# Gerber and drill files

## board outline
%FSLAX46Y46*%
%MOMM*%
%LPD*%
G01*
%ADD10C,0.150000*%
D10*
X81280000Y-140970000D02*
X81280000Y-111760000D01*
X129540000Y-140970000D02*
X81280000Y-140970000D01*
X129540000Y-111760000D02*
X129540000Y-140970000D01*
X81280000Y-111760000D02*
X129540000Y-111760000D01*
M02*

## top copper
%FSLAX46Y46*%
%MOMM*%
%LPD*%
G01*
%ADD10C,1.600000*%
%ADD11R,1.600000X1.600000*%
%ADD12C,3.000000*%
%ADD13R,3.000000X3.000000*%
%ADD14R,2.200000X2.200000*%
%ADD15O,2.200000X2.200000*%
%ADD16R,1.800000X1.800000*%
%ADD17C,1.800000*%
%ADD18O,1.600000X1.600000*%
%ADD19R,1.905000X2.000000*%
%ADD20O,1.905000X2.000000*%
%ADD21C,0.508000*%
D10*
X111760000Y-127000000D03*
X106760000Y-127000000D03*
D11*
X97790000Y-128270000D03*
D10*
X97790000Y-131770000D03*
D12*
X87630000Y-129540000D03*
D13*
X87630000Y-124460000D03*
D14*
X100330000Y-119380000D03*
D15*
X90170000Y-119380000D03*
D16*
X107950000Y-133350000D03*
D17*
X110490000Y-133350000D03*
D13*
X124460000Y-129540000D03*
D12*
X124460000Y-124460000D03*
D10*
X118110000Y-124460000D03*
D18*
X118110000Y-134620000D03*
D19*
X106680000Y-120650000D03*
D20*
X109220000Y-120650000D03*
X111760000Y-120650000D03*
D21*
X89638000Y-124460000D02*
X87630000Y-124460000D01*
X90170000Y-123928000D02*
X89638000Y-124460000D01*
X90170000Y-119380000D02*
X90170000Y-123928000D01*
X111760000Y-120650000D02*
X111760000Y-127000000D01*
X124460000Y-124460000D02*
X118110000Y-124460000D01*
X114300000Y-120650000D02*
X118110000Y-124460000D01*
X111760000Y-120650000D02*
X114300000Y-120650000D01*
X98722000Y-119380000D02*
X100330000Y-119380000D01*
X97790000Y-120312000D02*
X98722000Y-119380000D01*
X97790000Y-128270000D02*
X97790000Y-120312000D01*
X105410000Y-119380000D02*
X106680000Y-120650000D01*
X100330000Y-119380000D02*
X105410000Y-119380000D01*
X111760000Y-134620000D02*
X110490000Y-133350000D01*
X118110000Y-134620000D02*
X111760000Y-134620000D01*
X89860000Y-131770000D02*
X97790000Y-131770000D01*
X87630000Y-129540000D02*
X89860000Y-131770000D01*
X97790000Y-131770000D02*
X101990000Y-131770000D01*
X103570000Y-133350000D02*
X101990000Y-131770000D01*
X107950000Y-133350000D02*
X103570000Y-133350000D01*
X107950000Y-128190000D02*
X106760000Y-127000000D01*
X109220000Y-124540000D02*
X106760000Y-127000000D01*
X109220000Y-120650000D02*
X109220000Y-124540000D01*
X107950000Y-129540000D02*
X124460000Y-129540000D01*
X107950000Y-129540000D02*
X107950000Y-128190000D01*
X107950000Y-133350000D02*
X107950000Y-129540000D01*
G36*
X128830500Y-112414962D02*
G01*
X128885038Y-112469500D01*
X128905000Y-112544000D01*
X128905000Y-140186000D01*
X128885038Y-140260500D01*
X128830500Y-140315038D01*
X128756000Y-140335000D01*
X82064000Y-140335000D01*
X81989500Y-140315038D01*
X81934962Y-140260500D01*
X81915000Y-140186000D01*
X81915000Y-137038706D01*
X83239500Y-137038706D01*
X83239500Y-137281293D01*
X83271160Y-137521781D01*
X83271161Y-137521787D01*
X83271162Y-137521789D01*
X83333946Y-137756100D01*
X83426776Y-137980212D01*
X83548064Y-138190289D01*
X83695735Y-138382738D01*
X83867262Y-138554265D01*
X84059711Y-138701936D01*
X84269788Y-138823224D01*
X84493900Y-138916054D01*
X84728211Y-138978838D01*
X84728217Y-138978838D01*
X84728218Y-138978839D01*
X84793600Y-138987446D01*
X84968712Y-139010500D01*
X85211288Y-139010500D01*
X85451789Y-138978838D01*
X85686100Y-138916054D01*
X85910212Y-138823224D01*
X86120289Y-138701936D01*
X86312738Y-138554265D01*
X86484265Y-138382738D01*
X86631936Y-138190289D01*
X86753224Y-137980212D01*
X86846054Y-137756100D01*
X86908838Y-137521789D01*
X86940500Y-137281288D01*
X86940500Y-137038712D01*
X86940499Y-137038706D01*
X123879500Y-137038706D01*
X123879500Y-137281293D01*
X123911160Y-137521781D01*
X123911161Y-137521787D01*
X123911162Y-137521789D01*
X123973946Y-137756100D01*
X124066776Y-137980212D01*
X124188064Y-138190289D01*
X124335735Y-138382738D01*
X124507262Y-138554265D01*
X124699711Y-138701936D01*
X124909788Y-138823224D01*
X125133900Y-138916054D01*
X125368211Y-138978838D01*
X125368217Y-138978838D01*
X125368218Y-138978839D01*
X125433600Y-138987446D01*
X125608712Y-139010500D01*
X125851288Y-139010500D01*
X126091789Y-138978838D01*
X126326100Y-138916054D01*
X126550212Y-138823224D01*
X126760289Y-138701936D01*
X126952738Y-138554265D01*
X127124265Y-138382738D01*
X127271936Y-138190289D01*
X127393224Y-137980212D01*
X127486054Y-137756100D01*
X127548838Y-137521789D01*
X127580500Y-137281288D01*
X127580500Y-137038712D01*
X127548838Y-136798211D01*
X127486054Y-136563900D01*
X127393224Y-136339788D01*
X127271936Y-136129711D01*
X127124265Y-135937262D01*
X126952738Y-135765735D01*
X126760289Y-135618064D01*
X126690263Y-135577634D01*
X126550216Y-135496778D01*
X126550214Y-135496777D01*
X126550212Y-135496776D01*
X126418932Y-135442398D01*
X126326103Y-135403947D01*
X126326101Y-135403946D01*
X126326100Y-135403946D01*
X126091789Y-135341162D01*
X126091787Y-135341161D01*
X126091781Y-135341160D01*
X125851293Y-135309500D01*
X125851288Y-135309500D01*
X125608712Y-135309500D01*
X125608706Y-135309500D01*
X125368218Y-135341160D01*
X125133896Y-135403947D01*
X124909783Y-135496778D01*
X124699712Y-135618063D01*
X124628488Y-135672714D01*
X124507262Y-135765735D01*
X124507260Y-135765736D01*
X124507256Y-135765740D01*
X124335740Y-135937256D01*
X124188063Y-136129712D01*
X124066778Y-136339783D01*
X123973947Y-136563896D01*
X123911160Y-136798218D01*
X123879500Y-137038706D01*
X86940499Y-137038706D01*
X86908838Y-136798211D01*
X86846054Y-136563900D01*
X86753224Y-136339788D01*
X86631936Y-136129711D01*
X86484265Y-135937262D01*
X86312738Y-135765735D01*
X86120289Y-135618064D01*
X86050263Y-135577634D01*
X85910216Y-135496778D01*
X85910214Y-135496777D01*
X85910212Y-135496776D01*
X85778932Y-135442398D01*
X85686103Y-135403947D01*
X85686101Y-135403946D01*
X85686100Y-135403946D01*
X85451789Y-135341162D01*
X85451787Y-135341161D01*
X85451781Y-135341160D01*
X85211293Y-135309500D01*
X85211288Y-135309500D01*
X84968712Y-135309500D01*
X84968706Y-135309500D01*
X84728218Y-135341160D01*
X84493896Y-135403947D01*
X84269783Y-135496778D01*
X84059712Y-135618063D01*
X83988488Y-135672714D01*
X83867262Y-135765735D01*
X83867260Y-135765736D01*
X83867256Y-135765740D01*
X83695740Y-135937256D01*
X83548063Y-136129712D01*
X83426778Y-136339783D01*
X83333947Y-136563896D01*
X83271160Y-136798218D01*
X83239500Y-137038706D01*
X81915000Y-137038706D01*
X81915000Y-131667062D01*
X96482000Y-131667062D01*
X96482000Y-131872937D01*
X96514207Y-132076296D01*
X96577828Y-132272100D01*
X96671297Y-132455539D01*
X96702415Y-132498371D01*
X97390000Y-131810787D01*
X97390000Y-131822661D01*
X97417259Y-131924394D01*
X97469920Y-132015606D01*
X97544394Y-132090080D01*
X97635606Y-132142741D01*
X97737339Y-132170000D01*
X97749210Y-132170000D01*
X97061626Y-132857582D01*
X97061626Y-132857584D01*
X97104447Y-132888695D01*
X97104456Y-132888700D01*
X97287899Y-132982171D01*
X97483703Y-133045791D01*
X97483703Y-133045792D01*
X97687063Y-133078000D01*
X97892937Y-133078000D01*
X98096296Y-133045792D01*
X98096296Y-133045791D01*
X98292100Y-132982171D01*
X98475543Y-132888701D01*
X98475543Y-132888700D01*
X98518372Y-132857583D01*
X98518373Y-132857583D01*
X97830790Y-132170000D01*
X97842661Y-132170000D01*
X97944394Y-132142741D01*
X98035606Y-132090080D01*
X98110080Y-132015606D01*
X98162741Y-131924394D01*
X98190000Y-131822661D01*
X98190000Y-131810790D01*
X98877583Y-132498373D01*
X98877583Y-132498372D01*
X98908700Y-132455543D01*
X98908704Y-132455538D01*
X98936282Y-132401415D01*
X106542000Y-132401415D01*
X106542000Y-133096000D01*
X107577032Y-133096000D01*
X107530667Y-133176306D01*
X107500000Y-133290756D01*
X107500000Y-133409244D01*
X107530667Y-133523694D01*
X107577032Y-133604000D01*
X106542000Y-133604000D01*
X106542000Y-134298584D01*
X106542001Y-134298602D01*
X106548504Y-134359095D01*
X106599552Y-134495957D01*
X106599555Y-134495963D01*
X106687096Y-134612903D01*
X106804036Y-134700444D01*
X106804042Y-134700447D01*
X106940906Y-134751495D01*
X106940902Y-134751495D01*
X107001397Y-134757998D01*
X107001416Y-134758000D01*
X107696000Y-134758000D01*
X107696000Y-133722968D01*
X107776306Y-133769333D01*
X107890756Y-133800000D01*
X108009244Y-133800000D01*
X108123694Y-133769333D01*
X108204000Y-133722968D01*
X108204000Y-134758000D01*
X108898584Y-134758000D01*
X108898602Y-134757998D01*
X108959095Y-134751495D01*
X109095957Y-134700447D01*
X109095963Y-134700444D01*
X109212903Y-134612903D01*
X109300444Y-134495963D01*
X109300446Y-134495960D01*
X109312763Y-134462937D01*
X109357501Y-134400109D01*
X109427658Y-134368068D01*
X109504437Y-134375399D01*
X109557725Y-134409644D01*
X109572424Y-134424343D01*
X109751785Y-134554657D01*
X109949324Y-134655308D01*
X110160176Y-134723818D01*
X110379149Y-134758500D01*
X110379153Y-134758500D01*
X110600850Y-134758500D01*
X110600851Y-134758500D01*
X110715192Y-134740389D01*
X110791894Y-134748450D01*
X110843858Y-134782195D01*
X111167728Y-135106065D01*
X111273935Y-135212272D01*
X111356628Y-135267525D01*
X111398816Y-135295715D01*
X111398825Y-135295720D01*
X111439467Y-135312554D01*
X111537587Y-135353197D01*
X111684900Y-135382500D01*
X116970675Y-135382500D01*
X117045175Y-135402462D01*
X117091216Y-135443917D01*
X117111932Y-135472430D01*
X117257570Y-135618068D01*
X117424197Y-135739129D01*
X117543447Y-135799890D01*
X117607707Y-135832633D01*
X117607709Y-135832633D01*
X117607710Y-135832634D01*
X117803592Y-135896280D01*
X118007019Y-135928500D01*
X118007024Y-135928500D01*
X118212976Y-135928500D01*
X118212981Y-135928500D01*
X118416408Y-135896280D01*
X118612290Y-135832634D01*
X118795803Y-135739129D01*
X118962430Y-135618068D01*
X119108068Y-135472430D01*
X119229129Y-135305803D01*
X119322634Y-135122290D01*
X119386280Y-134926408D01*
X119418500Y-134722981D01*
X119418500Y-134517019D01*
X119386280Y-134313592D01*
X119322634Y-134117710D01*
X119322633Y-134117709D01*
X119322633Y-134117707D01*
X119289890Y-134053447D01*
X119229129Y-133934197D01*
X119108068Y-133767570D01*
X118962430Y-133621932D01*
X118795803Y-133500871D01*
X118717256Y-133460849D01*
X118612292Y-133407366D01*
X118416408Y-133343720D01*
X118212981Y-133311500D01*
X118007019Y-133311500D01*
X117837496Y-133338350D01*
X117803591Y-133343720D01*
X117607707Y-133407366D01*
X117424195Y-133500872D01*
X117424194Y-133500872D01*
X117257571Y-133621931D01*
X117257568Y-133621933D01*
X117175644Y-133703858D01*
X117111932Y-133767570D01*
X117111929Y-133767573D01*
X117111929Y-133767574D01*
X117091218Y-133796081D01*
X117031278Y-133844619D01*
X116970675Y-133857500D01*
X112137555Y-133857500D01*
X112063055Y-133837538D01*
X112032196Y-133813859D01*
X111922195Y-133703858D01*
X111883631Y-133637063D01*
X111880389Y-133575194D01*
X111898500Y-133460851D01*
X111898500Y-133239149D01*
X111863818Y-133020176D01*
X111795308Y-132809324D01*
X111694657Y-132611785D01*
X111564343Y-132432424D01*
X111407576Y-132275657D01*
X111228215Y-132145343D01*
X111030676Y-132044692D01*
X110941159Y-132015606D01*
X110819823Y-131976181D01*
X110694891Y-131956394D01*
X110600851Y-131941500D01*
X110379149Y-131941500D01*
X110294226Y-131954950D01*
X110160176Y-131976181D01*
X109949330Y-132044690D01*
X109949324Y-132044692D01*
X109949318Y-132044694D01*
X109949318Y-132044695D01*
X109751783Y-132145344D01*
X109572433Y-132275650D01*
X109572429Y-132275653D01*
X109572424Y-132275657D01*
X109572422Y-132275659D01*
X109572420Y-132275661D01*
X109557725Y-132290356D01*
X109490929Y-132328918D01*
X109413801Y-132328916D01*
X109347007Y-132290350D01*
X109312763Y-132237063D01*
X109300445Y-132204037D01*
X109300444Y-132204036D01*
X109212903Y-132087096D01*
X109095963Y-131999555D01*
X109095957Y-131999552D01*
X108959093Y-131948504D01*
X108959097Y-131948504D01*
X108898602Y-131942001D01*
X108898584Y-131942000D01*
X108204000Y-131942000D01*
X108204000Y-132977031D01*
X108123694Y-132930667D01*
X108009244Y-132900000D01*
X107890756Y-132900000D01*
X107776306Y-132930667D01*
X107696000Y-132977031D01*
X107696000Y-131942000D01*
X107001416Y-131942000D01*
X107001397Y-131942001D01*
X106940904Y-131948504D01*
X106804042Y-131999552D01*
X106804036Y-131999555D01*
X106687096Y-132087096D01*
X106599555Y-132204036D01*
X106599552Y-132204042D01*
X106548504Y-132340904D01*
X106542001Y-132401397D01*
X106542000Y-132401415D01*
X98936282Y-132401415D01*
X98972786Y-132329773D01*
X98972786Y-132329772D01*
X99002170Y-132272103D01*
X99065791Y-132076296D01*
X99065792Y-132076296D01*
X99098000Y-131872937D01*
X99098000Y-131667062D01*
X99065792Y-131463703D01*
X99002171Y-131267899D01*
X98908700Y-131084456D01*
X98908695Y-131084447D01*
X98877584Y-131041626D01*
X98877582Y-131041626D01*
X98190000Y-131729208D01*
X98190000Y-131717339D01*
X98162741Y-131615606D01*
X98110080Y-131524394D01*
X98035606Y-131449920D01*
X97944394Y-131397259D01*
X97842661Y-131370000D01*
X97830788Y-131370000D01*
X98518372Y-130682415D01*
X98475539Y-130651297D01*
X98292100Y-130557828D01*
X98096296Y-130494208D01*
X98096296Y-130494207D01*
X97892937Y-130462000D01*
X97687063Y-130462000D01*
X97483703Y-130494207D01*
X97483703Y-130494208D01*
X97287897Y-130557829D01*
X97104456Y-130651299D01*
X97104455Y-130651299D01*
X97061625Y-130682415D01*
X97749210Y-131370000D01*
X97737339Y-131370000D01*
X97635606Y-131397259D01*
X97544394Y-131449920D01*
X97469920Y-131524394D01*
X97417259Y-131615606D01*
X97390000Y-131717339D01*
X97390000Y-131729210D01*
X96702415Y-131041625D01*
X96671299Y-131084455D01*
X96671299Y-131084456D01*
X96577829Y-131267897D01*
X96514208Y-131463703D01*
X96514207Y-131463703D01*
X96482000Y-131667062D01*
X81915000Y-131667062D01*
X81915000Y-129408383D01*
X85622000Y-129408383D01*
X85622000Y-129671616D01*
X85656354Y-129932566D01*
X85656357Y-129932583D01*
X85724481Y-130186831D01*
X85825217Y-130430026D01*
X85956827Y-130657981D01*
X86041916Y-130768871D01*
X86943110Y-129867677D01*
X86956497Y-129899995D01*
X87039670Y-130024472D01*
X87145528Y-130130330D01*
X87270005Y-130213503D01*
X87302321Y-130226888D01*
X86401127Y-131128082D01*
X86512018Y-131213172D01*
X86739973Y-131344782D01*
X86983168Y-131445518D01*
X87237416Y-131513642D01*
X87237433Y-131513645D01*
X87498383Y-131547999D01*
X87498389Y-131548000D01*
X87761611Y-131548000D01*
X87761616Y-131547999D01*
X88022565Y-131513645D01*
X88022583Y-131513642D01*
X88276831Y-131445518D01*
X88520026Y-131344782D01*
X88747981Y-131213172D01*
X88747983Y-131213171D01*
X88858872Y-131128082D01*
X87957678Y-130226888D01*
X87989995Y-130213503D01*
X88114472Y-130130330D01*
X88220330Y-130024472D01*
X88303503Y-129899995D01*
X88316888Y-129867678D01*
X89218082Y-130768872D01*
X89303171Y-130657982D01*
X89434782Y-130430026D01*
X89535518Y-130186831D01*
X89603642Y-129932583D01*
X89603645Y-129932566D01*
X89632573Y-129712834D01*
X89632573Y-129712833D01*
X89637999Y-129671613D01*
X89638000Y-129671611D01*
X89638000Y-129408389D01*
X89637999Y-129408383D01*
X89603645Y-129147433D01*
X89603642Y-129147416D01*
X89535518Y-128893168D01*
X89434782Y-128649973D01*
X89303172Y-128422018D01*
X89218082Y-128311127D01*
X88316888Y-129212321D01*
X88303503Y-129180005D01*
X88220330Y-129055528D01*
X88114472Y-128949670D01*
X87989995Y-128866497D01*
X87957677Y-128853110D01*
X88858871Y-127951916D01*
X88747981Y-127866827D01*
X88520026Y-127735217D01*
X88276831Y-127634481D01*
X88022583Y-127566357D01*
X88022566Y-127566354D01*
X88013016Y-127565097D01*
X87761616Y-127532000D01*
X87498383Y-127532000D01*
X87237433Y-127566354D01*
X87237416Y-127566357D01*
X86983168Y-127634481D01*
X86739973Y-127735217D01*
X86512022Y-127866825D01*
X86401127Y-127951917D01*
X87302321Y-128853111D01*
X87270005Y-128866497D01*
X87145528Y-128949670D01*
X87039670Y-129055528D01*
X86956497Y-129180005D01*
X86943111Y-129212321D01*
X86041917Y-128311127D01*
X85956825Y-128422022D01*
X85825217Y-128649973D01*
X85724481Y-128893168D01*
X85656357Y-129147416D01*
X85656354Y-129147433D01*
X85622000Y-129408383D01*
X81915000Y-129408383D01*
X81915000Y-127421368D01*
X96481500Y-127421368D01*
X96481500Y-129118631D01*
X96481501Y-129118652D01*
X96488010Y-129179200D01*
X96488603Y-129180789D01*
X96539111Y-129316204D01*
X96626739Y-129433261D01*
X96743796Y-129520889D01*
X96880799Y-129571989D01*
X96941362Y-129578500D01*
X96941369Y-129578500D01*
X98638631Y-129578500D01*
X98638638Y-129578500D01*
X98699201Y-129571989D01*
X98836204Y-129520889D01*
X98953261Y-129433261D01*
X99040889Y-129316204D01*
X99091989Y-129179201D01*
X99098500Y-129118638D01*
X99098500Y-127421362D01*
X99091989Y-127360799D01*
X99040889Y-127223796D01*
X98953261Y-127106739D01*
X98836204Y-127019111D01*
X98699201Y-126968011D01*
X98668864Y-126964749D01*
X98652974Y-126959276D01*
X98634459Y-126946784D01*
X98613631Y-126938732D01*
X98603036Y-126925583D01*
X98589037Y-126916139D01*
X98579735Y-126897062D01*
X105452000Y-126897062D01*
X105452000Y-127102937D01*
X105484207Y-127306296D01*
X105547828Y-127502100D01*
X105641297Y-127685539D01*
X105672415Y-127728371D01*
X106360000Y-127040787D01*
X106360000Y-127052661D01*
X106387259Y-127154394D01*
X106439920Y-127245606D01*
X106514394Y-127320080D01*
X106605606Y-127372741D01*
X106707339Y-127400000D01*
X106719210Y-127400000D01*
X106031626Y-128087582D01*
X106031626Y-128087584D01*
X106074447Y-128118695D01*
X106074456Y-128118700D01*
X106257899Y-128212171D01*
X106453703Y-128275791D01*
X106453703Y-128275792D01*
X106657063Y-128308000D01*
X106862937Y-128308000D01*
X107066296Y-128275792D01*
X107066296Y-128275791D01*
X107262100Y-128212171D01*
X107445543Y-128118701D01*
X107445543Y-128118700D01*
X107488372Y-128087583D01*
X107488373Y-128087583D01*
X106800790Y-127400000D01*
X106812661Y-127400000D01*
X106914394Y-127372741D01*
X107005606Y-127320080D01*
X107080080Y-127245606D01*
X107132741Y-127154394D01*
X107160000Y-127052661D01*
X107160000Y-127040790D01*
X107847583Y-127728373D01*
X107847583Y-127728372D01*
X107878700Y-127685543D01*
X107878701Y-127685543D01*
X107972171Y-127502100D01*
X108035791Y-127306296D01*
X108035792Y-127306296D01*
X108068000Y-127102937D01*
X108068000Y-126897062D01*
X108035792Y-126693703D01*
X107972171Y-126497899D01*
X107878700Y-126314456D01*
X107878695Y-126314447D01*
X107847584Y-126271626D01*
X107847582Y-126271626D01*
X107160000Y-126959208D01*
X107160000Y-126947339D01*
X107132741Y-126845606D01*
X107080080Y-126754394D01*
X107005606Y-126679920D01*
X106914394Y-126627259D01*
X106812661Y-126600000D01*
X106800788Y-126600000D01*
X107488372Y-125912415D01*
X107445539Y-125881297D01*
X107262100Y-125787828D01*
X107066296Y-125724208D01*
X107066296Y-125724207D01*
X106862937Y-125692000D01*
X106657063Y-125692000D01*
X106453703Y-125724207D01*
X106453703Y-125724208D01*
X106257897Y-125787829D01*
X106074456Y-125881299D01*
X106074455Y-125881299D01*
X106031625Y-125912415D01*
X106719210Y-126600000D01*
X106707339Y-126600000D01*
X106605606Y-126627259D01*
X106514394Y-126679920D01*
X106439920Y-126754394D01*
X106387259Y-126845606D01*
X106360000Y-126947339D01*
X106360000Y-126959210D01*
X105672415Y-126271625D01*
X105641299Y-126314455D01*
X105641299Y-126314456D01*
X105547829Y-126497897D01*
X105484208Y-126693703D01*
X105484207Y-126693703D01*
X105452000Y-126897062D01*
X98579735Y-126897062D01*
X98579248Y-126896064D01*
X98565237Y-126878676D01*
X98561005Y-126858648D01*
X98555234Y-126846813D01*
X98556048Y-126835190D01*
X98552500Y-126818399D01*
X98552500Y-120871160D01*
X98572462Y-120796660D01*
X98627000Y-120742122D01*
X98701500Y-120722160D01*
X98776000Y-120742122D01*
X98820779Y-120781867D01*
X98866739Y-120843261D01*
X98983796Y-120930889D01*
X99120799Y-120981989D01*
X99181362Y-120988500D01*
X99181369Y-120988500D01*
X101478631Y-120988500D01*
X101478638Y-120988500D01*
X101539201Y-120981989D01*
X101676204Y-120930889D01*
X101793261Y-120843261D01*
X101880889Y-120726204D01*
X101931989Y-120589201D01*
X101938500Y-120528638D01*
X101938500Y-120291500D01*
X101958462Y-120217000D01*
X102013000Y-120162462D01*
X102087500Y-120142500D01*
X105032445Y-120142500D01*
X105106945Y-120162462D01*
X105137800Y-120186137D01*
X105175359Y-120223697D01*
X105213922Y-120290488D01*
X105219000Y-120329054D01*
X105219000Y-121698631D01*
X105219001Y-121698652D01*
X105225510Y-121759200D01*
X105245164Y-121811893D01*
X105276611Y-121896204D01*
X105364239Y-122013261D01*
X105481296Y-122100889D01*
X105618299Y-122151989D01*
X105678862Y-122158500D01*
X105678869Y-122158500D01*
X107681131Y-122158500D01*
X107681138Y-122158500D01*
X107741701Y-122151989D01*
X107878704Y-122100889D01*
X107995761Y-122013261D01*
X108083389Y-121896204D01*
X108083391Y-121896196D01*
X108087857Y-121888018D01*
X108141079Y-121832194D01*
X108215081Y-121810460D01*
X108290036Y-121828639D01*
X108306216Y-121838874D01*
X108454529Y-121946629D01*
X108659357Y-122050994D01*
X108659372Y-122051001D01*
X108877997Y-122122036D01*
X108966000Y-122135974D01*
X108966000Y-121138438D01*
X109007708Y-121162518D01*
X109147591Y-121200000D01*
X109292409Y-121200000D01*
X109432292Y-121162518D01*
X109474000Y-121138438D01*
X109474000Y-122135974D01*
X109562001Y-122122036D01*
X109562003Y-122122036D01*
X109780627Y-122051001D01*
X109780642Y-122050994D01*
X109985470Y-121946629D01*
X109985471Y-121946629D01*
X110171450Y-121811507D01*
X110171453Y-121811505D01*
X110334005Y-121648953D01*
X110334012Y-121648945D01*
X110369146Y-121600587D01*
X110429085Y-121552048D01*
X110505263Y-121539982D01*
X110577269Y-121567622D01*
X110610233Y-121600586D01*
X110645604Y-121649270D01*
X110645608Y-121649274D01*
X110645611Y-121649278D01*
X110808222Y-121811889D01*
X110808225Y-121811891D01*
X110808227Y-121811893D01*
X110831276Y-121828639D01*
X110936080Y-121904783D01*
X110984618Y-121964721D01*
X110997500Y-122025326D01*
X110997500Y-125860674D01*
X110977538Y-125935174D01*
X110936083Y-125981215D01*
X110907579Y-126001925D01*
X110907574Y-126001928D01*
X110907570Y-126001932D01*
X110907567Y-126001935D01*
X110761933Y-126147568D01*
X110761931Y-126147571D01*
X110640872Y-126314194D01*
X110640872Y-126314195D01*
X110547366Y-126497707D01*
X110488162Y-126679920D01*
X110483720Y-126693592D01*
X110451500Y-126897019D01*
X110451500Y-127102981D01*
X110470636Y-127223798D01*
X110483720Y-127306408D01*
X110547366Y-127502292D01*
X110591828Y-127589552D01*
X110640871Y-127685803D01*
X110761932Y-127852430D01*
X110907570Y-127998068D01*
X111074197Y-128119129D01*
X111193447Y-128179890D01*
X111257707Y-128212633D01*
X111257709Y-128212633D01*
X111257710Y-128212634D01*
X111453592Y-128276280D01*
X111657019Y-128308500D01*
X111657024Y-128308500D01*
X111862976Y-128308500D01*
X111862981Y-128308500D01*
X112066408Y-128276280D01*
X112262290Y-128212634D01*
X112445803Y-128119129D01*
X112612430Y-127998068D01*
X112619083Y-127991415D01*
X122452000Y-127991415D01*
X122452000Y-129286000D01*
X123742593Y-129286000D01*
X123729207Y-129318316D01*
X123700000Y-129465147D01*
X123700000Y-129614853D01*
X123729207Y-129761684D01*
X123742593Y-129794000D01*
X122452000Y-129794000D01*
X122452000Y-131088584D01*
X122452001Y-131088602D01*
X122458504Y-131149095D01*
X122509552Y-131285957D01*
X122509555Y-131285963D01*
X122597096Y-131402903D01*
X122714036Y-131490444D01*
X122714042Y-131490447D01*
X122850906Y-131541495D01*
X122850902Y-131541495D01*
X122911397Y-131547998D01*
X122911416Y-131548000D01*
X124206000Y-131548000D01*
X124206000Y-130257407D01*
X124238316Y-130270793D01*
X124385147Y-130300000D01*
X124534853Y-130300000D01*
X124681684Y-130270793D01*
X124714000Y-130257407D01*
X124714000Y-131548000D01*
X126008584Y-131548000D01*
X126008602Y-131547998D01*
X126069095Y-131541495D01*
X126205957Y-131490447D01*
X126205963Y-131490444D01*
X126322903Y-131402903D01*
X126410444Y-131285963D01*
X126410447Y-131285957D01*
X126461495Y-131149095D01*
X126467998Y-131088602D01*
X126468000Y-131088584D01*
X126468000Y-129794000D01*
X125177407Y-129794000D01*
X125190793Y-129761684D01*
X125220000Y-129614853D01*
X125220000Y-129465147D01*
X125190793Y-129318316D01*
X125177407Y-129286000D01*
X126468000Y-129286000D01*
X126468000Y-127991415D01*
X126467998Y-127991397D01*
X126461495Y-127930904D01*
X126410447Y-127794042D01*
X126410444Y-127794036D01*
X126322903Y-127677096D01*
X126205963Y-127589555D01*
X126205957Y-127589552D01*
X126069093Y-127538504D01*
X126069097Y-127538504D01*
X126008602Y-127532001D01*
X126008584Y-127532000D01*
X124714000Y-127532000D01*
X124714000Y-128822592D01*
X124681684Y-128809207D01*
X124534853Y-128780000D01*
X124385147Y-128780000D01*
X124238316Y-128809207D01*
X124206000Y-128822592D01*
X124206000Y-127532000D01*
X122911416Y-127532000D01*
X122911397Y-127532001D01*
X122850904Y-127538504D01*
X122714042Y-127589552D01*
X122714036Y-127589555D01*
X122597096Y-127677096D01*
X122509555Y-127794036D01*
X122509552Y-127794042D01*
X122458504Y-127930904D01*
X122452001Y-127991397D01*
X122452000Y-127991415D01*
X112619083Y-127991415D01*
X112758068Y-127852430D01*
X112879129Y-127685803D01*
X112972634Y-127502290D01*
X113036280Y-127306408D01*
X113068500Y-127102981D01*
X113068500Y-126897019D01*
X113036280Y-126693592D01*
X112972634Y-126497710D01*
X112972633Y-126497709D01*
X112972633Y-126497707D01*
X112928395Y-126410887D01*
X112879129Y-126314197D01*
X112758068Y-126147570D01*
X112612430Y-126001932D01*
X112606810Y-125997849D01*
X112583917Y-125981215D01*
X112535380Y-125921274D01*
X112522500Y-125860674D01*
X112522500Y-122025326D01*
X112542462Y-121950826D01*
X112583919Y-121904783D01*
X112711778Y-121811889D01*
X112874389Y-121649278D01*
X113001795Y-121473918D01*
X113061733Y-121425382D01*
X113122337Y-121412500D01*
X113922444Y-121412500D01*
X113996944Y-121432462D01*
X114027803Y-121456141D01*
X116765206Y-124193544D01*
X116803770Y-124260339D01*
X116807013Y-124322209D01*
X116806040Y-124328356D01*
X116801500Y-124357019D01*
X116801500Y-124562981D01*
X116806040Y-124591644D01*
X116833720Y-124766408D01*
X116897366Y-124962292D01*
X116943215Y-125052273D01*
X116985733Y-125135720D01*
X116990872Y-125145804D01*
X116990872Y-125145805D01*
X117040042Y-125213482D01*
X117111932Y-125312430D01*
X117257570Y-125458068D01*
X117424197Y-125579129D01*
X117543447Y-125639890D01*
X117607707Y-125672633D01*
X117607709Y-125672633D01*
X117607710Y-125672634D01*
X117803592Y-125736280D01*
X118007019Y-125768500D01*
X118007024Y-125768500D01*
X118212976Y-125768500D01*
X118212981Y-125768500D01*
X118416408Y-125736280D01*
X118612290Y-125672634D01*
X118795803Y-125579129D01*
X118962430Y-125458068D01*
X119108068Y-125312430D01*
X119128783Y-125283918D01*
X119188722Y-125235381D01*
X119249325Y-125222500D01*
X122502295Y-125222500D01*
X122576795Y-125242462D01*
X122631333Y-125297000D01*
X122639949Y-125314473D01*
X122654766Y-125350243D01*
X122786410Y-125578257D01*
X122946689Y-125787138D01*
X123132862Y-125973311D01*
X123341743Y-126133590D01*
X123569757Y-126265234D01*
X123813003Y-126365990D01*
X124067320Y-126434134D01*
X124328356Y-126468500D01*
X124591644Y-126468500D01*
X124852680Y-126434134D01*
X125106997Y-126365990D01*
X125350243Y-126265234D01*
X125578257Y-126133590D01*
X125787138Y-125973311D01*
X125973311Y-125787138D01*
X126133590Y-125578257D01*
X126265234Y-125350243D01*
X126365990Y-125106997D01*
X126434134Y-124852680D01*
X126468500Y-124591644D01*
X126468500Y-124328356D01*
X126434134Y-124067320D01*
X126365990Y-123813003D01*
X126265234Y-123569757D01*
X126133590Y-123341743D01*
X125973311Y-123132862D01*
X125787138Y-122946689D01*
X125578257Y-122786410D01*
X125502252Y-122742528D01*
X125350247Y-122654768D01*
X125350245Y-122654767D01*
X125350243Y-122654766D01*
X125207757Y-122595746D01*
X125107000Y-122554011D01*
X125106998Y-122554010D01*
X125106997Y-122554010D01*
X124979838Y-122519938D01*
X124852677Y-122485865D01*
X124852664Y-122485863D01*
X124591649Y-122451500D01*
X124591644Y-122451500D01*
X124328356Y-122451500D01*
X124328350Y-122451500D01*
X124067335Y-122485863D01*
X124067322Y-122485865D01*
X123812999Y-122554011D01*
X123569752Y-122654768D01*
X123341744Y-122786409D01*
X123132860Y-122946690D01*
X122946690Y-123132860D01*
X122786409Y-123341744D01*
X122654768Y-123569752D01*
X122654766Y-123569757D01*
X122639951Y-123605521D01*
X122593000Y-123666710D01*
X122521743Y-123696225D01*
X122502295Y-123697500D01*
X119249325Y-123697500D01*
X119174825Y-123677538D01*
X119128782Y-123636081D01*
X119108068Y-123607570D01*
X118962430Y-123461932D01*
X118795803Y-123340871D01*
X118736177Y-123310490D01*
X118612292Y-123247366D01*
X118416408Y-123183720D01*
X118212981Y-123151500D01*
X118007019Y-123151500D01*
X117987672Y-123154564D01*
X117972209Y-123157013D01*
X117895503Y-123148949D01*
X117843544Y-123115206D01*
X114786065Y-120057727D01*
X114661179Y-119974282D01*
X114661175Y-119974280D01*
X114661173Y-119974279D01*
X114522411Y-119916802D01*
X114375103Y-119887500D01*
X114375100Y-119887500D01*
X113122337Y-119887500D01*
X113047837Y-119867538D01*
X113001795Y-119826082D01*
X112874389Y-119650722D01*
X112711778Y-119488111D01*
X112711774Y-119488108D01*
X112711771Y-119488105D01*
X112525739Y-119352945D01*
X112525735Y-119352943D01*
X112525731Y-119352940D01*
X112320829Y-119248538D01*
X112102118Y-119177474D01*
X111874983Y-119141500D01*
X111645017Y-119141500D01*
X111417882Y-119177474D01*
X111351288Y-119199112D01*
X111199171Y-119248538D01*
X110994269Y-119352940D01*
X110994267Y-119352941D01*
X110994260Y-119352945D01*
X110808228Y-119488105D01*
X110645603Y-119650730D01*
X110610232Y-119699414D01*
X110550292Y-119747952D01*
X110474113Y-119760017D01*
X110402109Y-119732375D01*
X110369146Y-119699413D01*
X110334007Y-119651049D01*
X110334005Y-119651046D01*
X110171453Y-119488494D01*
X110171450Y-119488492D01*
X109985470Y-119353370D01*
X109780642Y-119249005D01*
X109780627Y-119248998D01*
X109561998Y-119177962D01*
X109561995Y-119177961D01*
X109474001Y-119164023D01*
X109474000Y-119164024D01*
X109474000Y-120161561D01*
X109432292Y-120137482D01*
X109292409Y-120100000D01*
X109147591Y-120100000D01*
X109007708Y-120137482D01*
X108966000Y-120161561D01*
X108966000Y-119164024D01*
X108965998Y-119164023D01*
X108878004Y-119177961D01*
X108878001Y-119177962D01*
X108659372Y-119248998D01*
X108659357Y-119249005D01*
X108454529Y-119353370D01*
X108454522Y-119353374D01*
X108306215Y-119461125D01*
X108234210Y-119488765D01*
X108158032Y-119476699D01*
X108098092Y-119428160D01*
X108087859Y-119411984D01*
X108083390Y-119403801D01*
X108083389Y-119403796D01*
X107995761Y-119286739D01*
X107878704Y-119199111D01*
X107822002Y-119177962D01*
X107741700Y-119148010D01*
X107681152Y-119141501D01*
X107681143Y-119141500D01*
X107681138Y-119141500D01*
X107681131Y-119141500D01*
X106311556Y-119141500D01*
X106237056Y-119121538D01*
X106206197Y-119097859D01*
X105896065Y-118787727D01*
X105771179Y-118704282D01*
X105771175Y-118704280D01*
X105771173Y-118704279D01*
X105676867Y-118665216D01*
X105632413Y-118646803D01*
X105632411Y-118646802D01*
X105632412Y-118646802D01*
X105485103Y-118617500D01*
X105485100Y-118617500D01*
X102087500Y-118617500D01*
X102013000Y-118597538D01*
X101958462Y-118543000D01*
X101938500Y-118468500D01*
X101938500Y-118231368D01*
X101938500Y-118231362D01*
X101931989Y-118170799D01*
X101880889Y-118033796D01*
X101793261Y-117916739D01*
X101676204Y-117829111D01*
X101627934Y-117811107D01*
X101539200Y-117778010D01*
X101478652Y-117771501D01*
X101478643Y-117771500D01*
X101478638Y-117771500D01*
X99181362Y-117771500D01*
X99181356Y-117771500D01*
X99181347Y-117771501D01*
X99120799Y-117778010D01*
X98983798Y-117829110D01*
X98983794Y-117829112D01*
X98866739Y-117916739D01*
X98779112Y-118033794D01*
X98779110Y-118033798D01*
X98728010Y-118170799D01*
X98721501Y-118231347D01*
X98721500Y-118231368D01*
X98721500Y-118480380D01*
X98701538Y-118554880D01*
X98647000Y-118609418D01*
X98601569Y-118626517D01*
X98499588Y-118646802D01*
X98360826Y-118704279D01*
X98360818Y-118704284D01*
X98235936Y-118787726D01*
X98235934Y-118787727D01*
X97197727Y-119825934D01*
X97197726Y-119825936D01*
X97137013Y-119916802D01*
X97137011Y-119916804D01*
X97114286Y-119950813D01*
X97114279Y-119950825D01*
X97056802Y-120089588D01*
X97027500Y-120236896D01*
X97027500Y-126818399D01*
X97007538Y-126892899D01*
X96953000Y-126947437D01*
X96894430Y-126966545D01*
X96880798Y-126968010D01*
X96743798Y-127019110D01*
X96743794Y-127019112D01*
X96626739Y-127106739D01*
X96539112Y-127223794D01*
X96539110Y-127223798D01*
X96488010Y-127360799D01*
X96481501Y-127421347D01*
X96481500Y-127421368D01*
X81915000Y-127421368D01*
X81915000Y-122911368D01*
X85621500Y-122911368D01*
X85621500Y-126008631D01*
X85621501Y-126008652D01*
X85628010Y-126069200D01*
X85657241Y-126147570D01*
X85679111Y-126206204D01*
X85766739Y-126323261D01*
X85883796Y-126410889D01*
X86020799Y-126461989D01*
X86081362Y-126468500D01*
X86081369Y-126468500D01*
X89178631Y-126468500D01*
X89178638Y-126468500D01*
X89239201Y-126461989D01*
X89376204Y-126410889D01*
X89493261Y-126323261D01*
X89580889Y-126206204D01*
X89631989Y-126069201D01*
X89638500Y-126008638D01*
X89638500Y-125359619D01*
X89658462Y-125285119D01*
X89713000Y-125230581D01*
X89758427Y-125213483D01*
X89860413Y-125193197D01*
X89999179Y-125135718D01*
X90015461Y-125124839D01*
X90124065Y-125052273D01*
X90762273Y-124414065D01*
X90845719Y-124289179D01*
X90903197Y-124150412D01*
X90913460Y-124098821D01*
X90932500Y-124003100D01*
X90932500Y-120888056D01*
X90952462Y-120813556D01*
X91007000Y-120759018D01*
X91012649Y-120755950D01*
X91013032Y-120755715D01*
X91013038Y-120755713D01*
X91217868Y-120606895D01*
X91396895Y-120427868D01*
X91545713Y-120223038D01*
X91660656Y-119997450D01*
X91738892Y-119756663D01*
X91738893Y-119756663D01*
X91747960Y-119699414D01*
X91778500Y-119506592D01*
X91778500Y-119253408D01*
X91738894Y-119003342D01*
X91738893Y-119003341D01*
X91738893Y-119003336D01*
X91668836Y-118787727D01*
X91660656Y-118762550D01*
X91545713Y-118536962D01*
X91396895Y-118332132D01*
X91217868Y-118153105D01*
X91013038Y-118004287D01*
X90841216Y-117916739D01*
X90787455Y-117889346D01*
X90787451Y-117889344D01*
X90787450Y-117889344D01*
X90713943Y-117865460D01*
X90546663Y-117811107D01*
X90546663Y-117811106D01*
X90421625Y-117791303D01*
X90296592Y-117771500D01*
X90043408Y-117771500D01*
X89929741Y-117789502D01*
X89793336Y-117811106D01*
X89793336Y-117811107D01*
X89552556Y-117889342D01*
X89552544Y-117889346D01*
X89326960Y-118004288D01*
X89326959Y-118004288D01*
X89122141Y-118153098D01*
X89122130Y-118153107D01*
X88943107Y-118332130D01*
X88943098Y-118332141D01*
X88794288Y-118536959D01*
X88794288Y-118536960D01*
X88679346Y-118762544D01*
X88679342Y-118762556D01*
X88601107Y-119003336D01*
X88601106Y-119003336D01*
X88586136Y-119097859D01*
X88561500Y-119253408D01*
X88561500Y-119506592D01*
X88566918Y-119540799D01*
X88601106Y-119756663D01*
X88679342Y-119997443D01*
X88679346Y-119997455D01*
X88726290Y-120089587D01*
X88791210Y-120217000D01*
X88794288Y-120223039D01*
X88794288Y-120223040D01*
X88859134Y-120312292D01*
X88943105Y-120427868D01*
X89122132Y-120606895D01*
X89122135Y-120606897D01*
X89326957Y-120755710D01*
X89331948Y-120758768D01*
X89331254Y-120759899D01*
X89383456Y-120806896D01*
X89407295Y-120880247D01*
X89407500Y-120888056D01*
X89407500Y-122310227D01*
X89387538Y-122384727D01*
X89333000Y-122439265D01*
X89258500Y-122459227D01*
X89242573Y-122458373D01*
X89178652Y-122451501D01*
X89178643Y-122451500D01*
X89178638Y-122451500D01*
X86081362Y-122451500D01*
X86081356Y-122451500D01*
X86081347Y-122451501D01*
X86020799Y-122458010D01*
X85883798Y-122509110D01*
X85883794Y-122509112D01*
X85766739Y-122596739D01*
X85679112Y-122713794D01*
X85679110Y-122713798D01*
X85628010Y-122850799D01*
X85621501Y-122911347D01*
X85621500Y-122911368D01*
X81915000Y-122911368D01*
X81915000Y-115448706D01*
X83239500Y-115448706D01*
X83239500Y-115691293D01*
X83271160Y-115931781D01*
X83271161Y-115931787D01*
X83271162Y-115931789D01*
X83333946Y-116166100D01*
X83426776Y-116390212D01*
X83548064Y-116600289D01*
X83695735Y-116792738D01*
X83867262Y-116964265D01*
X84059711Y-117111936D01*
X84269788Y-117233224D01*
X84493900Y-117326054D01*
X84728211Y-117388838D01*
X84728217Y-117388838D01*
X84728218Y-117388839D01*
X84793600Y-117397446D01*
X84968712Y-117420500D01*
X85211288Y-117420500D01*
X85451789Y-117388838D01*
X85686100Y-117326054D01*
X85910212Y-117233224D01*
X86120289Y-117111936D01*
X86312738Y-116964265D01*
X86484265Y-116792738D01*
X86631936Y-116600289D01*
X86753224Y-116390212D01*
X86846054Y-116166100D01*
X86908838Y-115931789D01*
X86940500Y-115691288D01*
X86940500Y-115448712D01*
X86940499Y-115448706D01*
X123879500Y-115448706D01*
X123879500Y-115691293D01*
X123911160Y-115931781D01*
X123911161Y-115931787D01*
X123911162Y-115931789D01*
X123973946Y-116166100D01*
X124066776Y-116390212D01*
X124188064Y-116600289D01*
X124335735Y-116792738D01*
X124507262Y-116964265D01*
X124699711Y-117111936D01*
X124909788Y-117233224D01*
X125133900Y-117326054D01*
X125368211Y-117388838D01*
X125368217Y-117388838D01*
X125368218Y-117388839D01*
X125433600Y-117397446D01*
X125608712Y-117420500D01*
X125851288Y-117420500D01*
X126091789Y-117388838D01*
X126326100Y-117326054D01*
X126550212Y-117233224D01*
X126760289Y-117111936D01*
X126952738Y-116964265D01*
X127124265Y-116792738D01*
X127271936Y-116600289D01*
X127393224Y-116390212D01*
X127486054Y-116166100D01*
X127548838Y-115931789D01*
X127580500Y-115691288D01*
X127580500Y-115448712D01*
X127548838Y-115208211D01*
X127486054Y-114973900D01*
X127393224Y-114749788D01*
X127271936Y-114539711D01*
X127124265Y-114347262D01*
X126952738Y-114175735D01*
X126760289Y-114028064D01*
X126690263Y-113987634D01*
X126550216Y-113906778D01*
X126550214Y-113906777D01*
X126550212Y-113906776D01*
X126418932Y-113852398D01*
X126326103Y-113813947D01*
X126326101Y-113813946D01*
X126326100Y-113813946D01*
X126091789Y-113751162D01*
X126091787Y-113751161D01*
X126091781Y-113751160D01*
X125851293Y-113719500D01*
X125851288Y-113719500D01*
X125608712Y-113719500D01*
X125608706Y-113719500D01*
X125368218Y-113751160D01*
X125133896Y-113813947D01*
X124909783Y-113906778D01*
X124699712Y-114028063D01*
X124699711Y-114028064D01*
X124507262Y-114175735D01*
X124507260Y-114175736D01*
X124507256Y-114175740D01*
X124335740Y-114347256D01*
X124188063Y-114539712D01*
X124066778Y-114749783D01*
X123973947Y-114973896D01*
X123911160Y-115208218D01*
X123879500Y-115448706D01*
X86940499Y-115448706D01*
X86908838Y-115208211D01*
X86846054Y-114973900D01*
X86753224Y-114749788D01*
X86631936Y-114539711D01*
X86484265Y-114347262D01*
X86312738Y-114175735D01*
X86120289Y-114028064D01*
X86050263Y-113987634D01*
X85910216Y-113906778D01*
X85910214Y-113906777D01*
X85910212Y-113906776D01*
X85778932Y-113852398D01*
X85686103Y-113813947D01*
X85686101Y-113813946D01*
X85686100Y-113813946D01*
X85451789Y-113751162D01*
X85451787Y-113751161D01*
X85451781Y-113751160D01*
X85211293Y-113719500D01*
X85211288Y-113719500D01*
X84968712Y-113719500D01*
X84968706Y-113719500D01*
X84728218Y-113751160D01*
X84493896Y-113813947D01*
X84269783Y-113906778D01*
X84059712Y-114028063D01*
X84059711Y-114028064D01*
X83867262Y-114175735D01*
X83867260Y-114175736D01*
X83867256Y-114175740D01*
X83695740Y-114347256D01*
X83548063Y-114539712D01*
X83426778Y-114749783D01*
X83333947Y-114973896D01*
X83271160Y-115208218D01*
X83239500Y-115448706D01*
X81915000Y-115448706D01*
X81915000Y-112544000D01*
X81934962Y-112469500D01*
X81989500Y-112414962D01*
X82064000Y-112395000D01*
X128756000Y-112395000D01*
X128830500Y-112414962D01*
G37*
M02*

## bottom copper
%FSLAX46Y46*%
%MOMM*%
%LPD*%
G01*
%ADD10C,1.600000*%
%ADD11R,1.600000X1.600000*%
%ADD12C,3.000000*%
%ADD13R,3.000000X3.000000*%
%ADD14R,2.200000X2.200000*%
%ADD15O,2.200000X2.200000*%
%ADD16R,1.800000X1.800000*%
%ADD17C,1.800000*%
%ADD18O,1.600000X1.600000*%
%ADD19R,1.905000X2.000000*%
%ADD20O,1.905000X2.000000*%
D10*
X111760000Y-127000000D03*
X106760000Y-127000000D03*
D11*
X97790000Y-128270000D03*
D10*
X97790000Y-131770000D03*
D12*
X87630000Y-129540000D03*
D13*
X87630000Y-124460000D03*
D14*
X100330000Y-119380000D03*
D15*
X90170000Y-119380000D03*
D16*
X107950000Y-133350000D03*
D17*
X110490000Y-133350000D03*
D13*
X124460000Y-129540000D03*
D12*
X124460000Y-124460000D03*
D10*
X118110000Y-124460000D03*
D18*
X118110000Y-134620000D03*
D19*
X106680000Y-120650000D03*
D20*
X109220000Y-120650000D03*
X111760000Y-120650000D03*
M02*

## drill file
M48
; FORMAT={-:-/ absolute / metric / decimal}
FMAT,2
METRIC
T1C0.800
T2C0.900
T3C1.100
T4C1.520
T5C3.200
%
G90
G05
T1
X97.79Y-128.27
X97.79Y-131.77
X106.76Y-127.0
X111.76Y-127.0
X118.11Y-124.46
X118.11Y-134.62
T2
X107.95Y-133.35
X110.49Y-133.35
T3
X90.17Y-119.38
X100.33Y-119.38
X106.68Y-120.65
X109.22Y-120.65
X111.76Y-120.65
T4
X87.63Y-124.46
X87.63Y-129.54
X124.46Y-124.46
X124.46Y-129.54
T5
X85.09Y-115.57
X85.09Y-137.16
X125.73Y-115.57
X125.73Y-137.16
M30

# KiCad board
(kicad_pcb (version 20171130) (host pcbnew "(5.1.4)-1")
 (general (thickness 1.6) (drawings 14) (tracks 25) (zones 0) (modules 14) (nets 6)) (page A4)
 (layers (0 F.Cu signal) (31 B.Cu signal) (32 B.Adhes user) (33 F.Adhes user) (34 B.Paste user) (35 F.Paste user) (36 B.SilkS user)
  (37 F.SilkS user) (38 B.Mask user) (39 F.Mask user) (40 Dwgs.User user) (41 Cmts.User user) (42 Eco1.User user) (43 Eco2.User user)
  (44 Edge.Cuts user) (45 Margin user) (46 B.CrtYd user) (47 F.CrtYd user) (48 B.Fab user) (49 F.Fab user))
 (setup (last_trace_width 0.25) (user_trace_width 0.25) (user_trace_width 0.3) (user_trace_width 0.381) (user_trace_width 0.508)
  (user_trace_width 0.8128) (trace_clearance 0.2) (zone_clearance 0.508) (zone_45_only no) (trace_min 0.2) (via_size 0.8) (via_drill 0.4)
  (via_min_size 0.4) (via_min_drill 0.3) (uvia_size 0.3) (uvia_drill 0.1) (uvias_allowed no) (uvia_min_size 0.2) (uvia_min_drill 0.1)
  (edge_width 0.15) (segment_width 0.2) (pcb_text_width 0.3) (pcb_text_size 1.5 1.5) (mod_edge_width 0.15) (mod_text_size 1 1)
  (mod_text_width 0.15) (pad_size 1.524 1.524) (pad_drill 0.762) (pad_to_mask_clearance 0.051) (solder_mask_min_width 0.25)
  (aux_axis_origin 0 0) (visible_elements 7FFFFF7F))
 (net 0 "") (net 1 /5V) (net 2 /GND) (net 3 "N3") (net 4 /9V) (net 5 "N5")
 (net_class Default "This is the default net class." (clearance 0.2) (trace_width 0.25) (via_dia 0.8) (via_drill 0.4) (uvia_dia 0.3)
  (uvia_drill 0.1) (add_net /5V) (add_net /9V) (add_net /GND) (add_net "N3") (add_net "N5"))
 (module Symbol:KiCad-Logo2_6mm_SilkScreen (layer B.Cu) (at 97.79 137.795)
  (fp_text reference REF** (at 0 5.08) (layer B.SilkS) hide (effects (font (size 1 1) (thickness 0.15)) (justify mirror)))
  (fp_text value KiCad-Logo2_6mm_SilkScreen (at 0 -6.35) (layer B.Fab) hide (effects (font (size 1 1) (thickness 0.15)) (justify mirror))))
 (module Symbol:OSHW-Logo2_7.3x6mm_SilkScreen (layer B.Cu) (at 118.11 115.57)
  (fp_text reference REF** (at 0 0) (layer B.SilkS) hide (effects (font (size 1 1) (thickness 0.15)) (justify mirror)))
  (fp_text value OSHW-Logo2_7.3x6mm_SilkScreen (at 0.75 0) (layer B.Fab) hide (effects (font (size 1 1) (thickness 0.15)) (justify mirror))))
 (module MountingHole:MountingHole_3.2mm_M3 (layer F.Cu) (at 85.09 137.16)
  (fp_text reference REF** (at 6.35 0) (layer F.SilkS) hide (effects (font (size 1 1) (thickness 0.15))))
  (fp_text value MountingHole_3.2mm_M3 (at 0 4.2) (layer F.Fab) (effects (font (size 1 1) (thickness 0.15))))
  (pad 1 np_thru_hole circle (at 0 0) (size 3.2 3.2) (drill 3.2) (layers *.Cu *.Mask)))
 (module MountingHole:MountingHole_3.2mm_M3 (layer F.Cu) (at 85.09 115.57)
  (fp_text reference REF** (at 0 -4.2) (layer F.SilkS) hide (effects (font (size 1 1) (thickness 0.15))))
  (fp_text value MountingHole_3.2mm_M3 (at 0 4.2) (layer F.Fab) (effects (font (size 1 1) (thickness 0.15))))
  (pad 1 np_thru_hole circle (at 0 0) (size 3.2 3.2) (drill 3.2) (layers *.Cu *.Mask)))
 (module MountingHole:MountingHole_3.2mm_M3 (layer F.Cu) (at 125.73 137.16)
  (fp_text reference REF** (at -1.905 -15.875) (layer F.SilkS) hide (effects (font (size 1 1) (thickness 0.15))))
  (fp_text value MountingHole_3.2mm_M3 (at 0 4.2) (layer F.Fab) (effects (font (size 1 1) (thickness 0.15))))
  (pad 1 np_thru_hole circle (at 0 0) (size 3.2 3.2) (drill 3.2) (layers *.Cu *.Mask)))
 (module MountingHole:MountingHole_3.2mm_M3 (layer F.Cu) (at 125.73 115.57)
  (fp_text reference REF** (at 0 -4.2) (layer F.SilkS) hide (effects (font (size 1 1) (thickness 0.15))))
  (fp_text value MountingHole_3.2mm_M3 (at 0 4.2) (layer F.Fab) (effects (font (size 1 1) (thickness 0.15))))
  (pad 1 np_thru_hole circle (at 0 0) (size 3.2 3.2) (drill 3.2) (layers *.Cu *.Mask)))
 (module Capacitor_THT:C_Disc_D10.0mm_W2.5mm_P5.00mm (layer F.Cu) (at 111.76 127 180)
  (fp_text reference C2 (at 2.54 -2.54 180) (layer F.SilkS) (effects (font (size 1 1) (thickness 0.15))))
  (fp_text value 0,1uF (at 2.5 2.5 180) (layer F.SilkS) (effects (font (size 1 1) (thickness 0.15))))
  (pad 1 thru_hole circle (at 0 0 180) (size 1.6 1.6) (drill 0.8) (layers *.Cu *.Mask) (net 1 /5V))
  (pad 2 thru_hole circle (at 5 0 180) (size 1.6 1.6) (drill 0.8) (layers *.Cu *.Mask) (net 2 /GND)))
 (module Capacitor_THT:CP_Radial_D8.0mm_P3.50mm (layer F.Cu) (at 97.79 128.27 270)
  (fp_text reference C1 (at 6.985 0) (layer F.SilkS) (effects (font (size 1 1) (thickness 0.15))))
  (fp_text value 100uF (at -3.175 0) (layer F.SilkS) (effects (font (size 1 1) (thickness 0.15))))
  (pad 1 thru_hole rect (at 0 0 270) (size 1.6 1.6) (drill 0.8) (layers *.Cu *.Mask) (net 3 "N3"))
  (pad 2 thru_hole circle (at 3.5 0 270) (size 1.6 1.6) (drill 0.8) (layers *.Cu *.Mask) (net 2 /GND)))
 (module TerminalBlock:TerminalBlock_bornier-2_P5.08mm (layer F.Cu) (at 87.63 124.46 270)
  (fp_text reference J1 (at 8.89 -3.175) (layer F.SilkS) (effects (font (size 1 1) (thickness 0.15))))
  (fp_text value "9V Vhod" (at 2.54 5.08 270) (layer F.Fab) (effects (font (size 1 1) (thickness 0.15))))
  (pad 2 thru_hole circle (at 5.08 0 270) (size 3 3) (drill 1.52) (layers *.Cu *.Mask) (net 2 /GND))
  (pad 1 thru_hole rect (at 0 0 270) (size 3 3) (drill 1.52) (layers *.Cu *.Mask) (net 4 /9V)))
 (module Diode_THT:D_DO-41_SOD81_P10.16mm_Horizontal (layer F.Cu) (at 100.33 119.38 180)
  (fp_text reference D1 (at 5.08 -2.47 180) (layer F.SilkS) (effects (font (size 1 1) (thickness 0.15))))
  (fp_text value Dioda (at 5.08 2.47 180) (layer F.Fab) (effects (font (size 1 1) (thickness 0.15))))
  (pad 1 thru_hole rect (at 0 0 180) (size 2.2 2.2) (drill 1.1) (layers *.Cu *.Mask) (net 3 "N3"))
  (pad 2 thru_hole oval (at 10.16 0 180) (size 2.2 2.2) (drill 1.1) (layers *.Cu *.Mask) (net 4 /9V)))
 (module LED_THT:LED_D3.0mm (layer F.Cu) (at 107.95 133.35)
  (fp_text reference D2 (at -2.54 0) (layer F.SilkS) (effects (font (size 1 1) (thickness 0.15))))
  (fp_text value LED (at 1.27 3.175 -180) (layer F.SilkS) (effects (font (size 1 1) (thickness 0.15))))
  (pad 1 thru_hole rect (at 0 0) (size 1.8 1.8) (drill 0.9) (layers *.Cu *.Mask) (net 2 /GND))
  (pad 2 thru_hole circle (at 2.54 0) (size 1.8 1.8) (drill 0.9) (layers *.Cu *.Mask) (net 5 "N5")))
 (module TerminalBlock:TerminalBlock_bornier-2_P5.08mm (layer F.Cu) (at 124.46 129.54 90)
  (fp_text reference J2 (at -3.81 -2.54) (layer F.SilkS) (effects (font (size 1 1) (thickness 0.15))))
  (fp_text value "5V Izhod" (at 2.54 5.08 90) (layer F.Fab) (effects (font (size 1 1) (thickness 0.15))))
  (pad 1 thru_hole rect (at 0 0 90) (size 3 3) (drill 1.52) (layers *.Cu *.Mask) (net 2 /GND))
  (pad 2 thru_hole circle (at 5.08 0 90) (size 3 3) (drill 1.52) (layers *.Cu *.Mask) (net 1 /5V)))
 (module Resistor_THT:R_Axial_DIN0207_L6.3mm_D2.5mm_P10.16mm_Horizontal (layer F.Cu) (at 118.11 124.46 270)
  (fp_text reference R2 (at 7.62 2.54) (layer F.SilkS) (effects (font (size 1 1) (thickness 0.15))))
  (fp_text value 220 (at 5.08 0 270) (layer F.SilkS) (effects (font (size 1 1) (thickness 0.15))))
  (pad 1 thru_hole circle (at 0 0 270) (size 1.6 1.6) (drill 0.8) (layers *.Cu *.Mask) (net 1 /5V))
  (pad 2 thru_hole oval (at 10.16 0 270) (size 1.6 1.6) (drill 0.8) (layers *.Cu *.Mask) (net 5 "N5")))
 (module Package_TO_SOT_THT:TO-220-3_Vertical (layer F.Cu) (at 106.68 120.65)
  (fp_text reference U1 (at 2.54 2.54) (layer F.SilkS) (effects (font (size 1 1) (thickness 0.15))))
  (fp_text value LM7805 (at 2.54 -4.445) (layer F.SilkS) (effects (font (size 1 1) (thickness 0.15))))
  (pad 1 thru_hole rect (at 0 0) (size 1.905 2) (drill 1.1) (layers *.Cu *.Mask) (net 3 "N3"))
  (pad 2 thru_hole oval (at 2.54 0) (size 1.905 2) (drill 1.1) (layers *.Cu *.Mask) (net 2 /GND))
  (pad 3 thru_hole oval (at 5.08 0) (size 1.905 2) (drill 1.1) (layers *.Cu *.Mask) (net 1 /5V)))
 (gr_line (start 81.28 140.97) (end 81.28 111.76) (layer Edge.Cuts) (width 0.15))
 (gr_line (start 129.54 140.97) (end 81.28 140.97) (layer Edge.Cuts) (width 0.15))
 (gr_line (start 129.54 111.76) (end 129.54 140.97) (layer Edge.Cuts) (width 0.15))
 (gr_line (start 81.28 111.76) (end 129.54 111.76) (layer Edge.Cuts) (width 0.15))
 (segment (start 89.638 124.46) (end 87.63 124.46) (width 0.508) (layer F.Cu) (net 4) (status 20))
 (segment (start 90.17 123.928) (end 89.638 124.46) (width 0.508) (layer F.Cu) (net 4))
 (segment (start 90.17 119.38) (end 90.17 123.928) (width 0.508) (layer F.Cu) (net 4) (status 10))
 (segment (start 111.76 120.65) (end 111.76 127) (width 0.508) (layer F.Cu) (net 1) (status 30))
 (segment (start 124.46 124.46) (end 118.11 124.46) (width 0.508) (layer F.Cu) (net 1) (status 30))
 (segment (start 114.3 120.65) (end 118.11 124.46) (width 0.508) (layer F.Cu) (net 1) (status 20))
 (segment (start 111.76 120.65) (end 114.3 120.65) (width 0.508) (layer F.Cu) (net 1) (status 10))
 (segment (start 98.722 119.38) (end 100.33 119.38) (width 0.508) (layer F.Cu) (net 3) (status 20))
 (segment (start 97.79 120.312) (end 98.722 119.38) (width 0.508) (layer F.Cu) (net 3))
 (segment (start 97.79 128.27) (end 97.79 120.312) (width 0.508) (layer F.Cu) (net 3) (status 10))
 (segment (start 105.41 119.38) (end 106.68 120.65) (width 0.508) (layer F.Cu) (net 3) (status 20))
 (segment (start 100.33 119.38) (end 105.41 119.38) (width 0.508) (layer F.Cu) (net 3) (status 10))
 (segment (start 111.76 134.62) (end 110.49 133.35) (width 0.508) (layer F.Cu) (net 5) (status 20))
 (segment (start 118.11 134.62) (end 111.76 134.62) (width 0.508) (layer F.Cu) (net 5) (status 10))
 (segment (start 89.86 131.77) (end 97.79 131.77) (width 0.508) (layer F.Cu) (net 2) (status 20))
 (segment (start 87.63 129.54) (end 89.86 131.77) (width 0.508) (layer F.Cu) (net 2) (status 10))
 (segment (start 97.79 131.77) (end 101.99 131.77) (width 0.508) (layer F.Cu) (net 2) (status 10))
 (segment (start 103.57 133.35) (end 101.99 131.77) (width 0.508) (layer F.Cu) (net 2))
 (segment (start 107.95 133.35) (end 103.57 133.35) (width 0.508) (layer F.Cu) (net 2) (status 10))
 (segment (start 107.95 128.19) (end 106.76 127) (width 0.508) (layer F.Cu) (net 2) (status 20))
 (segment (start 109.22 124.54) (end 106.76 127) (width 0.508) (layer F.Cu) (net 2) (status 20))
 (segment (start 109.22 120.65) (end 109.22 124.54) (width 0.508) (layer F.Cu) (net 2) (status 10))
 (segment (start 107.95 129.54) (end 124.46 129.54) (width 0.508) (layer F.Cu) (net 2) (status 20))
 (segment (start 107.95 129.54) (end 107.95 128.19) (width 0.508) (layer F.Cu) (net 2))
 (segment (start 107.95 133.35) (end 107.95 129.54) (width 0.508) (layer F.Cu) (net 2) (status 10))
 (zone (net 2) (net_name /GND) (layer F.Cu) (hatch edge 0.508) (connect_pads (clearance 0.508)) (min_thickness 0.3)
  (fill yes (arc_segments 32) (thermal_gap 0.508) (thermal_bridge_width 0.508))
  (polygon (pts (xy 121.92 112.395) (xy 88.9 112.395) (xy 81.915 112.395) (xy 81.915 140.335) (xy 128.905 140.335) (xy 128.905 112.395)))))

